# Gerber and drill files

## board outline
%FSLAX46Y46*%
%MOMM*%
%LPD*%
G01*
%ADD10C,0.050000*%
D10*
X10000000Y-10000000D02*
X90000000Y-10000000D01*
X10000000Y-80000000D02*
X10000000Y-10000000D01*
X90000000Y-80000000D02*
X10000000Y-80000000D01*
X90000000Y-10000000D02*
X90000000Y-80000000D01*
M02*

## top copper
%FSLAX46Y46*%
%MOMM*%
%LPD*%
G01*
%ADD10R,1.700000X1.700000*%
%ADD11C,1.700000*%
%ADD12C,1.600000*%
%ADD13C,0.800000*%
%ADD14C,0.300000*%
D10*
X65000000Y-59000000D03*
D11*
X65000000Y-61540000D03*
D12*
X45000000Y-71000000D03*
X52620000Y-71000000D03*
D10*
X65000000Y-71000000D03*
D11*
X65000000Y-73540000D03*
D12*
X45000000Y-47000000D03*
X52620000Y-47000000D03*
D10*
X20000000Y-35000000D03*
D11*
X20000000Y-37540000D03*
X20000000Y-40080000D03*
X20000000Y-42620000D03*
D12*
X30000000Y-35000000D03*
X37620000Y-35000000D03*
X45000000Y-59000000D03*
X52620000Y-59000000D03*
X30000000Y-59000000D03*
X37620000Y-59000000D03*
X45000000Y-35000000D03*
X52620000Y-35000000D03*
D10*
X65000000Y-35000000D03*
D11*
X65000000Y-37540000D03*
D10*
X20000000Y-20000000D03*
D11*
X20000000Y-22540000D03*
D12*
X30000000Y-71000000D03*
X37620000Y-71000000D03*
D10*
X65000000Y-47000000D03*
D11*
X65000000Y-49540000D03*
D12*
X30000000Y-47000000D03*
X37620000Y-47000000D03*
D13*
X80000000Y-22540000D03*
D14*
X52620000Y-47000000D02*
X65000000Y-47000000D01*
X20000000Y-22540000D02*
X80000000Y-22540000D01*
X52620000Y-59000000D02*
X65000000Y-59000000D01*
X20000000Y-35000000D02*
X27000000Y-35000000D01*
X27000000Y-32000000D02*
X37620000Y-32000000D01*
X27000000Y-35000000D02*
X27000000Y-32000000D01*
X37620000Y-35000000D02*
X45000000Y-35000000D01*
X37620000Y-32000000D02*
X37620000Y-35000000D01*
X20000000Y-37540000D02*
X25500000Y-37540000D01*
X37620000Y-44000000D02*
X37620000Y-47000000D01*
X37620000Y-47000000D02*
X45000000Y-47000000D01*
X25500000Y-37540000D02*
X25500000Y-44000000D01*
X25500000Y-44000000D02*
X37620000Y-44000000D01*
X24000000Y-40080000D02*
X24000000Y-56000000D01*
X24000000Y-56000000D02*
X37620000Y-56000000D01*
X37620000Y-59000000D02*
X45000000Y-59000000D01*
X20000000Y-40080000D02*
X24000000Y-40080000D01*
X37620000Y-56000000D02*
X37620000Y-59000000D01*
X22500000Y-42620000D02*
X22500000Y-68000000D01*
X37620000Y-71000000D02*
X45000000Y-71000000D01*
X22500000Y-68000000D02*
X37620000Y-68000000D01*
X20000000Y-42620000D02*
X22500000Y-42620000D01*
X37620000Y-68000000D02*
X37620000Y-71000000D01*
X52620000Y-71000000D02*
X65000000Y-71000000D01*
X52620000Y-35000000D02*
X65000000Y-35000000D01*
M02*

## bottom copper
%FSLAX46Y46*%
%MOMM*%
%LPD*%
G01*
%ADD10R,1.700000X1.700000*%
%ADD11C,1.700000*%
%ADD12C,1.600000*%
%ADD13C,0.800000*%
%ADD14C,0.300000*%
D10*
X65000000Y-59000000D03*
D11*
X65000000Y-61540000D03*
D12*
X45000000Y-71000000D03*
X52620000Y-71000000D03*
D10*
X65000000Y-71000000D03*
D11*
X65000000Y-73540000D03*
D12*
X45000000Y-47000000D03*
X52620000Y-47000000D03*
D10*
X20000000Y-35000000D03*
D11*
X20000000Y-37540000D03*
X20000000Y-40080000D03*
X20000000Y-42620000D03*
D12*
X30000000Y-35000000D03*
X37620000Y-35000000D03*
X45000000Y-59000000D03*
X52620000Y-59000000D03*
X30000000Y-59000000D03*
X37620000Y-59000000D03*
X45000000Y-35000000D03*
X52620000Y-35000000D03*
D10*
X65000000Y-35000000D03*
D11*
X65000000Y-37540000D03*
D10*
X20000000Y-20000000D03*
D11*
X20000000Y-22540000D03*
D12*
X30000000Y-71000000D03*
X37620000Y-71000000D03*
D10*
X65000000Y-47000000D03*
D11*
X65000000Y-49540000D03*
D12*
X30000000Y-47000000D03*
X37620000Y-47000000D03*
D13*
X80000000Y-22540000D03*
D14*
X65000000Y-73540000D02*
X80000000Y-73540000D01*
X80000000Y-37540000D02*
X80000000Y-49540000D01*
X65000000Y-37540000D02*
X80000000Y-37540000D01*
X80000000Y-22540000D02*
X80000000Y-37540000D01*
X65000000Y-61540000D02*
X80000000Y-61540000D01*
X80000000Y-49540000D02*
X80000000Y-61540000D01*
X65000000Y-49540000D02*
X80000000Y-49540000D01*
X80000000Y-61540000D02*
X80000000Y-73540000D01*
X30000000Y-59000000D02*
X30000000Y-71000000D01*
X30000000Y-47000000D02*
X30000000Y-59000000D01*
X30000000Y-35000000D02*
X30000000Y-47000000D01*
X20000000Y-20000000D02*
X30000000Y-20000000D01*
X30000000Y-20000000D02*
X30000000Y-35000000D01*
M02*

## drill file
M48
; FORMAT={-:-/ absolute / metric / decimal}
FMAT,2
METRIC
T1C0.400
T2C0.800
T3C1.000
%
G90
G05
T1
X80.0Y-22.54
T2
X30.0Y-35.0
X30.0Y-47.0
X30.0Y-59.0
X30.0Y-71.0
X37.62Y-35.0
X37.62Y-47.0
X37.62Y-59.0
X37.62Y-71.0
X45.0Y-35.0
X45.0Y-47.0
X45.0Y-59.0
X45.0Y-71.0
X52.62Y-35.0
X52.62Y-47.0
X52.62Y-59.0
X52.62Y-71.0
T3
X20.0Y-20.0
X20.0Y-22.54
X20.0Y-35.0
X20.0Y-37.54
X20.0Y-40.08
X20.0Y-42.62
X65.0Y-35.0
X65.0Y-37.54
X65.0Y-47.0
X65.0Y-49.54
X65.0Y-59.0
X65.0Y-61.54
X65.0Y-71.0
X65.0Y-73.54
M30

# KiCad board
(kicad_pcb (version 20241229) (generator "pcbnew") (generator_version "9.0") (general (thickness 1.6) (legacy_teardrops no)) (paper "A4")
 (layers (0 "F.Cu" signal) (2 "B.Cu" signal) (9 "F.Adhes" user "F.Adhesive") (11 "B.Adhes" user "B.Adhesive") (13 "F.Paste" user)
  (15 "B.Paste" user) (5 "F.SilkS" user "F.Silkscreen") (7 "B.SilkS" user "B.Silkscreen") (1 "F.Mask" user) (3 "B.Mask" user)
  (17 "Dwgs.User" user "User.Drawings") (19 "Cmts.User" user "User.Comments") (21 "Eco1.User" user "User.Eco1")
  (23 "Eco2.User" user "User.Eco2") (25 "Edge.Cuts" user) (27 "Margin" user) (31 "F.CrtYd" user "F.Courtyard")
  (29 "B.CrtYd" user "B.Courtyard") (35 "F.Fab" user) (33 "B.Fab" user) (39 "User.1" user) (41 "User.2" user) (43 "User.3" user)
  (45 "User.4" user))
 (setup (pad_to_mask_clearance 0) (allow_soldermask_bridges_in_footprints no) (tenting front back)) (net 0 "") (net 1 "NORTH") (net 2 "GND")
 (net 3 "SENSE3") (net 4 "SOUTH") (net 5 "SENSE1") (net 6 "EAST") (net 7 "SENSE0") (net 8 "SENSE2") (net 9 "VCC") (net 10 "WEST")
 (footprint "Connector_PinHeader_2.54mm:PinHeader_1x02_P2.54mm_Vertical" (layer "F.Cu") (at 65 59)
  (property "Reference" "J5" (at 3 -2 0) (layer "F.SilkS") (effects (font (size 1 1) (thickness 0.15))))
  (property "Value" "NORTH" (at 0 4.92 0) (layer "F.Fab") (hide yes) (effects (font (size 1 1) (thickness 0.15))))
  (pad "1" thru_hole rect (at 0 0) (size 1.7 1.7) (drill 1) (layers "*.Cu" "*.Mask") (remove_unused_layers no) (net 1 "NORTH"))
  (pad "2" thru_hole circle (at 0 2.54) (size 1.7 1.7) (drill 1) (layers "*.Cu" "*.Mask") (remove_unused_layers no) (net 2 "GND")))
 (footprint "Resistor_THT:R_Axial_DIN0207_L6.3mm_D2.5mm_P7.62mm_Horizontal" (layer "F.Cu") (at 45 71)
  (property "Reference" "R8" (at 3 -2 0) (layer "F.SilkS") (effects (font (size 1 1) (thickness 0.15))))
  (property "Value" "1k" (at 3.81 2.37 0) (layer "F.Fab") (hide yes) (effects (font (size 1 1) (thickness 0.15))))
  (pad "1" thru_hole circle (at 0 0) (size 1.6 1.6) (drill 0.8) (layers "*.Cu" "*.Mask") (remove_unused_layers no) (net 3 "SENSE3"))
  (pad "2" thru_hole circle (at 7.62 0) (size 1.6 1.6) (drill 0.8) (layers "*.Cu" "*.Mask") (remove_unused_layers no) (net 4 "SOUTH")))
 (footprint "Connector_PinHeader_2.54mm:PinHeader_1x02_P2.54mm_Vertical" (layer "F.Cu") (at 65 71)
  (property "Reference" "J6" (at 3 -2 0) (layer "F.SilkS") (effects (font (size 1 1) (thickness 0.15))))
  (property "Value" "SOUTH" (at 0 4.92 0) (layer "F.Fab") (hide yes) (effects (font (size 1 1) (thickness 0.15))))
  (pad "1" thru_hole rect (at 0 0) (size 1.7 1.7) (drill 1) (layers "*.Cu" "*.Mask") (remove_unused_layers no) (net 4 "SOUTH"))
  (pad "2" thru_hole circle (at 0 2.54) (size 1.7 1.7) (drill 1) (layers "*.Cu" "*.Mask") (remove_unused_layers no) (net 2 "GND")))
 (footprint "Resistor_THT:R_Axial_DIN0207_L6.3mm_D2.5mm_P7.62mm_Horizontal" (layer "F.Cu") (at 45 47)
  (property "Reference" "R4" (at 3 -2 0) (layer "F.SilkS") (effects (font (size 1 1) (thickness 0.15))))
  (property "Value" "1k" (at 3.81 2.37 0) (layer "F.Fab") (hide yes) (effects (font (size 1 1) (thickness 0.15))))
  (pad "1" thru_hole circle (at 0 0) (size 1.6 1.6) (drill 0.8) (layers "*.Cu" "*.Mask") (remove_unused_layers no) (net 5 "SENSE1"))
  (pad "2" thru_hole circle (at 7.62 0) (size 1.6 1.6) (drill 0.8) (layers "*.Cu" "*.Mask") (remove_unused_layers no) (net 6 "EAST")))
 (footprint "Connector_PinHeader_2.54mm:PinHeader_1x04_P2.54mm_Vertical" (layer "F.Cu") (at 20 35)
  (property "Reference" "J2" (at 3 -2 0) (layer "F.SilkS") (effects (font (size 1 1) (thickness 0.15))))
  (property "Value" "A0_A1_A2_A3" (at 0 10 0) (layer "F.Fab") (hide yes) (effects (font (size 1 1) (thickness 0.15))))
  (pad "1" thru_hole rect (at 0 0) (size 1.7 1.7) (drill 1) (layers "*.Cu" "*.Mask") (remove_unused_layers no) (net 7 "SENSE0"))
  (pad "2" thru_hole circle (at 0 2.54) (size 1.7 1.7) (drill 1) (layers "*.Cu" "*.Mask") (remove_unused_layers no) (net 5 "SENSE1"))
  (pad "3" thru_hole circle (at 0 5.08) (size 1.7 1.7) (drill 1) (layers "*.Cu" "*.Mask") (remove_unused_layers no) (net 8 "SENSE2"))
  (pad "4" thru_hole circle (at 0 7.62) (size 1.7 1.7) (drill 1) (layers "*.Cu" "*.Mask") (remove_unused_layers no) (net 3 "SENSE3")))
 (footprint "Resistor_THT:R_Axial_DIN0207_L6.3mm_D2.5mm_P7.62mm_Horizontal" (layer "F.Cu") (at 30 35)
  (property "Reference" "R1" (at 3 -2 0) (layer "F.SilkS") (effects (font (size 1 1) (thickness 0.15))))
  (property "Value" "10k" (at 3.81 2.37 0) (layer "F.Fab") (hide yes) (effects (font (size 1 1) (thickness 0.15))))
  (pad "1" thru_hole circle (at 0 0) (size 1.6 1.6) (drill 0.8) (layers "*.Cu" "*.Mask") (remove_unused_layers no) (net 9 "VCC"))
  (pad "2" thru_hole circle (at 7.62 0) (size 1.6 1.6) (drill 0.8) (layers "*.Cu" "*.Mask") (remove_unused_layers no) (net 7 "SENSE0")))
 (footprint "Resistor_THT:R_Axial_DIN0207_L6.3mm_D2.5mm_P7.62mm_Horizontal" (layer "F.Cu") (at 45 59)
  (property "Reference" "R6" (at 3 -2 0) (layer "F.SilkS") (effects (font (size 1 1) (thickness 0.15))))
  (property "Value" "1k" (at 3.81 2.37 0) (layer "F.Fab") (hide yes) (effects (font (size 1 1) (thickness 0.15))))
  (pad "1" thru_hole circle (at 0 0) (size 1.6 1.6) (drill 0.8) (layers "*.Cu" "*.Mask") (remove_unused_layers no) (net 8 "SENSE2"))
  (pad "2" thru_hole circle (at 7.62 0) (size 1.6 1.6) (drill 0.8) (layers "*.Cu" "*.Mask") (remove_unused_layers no) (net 1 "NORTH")))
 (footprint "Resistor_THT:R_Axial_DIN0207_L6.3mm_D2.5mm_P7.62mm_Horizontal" (layer "F.Cu") (at 30 59)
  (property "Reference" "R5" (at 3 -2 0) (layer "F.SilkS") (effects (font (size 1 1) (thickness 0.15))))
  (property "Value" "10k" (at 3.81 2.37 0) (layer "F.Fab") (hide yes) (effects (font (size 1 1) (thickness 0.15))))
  (pad "1" thru_hole circle (at 0 0) (size 1.6 1.6) (drill 0.8) (layers "*.Cu" "*.Mask") (remove_unused_layers no) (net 9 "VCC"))
  (pad "2" thru_hole circle (at 7.62 0) (size 1.6 1.6) (drill 0.8) (layers "*.Cu" "*.Mask") (remove_unused_layers no) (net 8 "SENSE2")))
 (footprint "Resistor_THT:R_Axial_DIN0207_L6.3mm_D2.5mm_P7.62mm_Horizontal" (layer "F.Cu") (at 45 35)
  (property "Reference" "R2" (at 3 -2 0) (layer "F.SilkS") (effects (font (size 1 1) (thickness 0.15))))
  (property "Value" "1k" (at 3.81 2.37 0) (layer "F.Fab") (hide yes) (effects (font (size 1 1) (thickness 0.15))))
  (pad "1" thru_hole circle (at 0 0) (size 1.6 1.6) (drill 0.8) (layers "*.Cu" "*.Mask") (remove_unused_layers no) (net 7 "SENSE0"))
  (pad "2" thru_hole circle (at 7.62 0) (size 1.6 1.6) (drill 0.8) (layers "*.Cu" "*.Mask") (remove_unused_layers no) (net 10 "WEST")))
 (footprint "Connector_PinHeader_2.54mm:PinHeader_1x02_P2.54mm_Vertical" (layer "F.Cu") (at 65 35)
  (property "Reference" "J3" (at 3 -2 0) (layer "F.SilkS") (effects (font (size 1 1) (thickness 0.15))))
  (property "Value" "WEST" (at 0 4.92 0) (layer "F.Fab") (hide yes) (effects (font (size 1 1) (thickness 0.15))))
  (pad "1" thru_hole rect (at 0 0) (size 1.7 1.7) (drill 1) (layers "*.Cu" "*.Mask") (remove_unused_layers no) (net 10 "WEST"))
  (pad "2" thru_hole circle (at 0 2.54) (size 1.7 1.7) (drill 1) (layers "*.Cu" "*.Mask") (remove_unused_layers no) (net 2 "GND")))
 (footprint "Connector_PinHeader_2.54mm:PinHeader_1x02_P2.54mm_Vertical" (layer "F.Cu") (at 20 20)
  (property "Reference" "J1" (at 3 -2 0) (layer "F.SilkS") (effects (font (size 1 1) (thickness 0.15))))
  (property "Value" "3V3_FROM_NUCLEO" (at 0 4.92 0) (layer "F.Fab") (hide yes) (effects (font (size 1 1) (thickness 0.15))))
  (pad "1" thru_hole rect (at 0 0) (size 1.7 1.7) (drill 1) (layers "*.Cu" "*.Mask") (remove_unused_layers no) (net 9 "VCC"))
  (pad "2" thru_hole circle (at 0 2.54) (size 1.7 1.7) (drill 1) (layers "*.Cu" "*.Mask") (remove_unused_layers no) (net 2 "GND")))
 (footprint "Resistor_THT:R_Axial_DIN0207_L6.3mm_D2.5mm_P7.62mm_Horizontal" (layer "F.Cu") (at 30 71)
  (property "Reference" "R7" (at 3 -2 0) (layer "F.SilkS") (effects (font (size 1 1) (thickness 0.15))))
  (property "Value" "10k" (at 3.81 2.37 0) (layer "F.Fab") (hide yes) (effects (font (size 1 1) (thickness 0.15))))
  (pad "1" thru_hole circle (at 0 0) (size 1.6 1.6) (drill 0.8) (layers "*.Cu" "*.Mask") (remove_unused_layers no) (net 9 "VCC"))
  (pad "2" thru_hole circle (at 7.62 0) (size 1.6 1.6) (drill 0.8) (layers "*.Cu" "*.Mask") (remove_unused_layers no) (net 3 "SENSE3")))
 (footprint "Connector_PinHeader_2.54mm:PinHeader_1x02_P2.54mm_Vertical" (layer "F.Cu") (at 65 47)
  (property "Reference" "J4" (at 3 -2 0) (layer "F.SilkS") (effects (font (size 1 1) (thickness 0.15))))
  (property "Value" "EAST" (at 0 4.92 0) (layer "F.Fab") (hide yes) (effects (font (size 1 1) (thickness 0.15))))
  (pad "1" thru_hole rect (at 0 0) (size 1.7 1.7) (drill 1) (layers "*.Cu" "*.Mask") (remove_unused_layers no) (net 6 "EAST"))
  (pad "2" thru_hole circle (at 0 2.54) (size 1.7 1.7) (drill 1) (layers "*.Cu" "*.Mask") (remove_unused_layers no) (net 2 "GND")))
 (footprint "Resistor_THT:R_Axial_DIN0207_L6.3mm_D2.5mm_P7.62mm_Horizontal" (layer "F.Cu") (at 30 47)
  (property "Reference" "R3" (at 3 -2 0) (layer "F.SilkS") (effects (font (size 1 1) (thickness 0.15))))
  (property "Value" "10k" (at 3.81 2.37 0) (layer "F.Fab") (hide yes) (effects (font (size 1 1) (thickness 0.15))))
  (pad "1" thru_hole circle (at 0 0) (size 1.6 1.6) (drill 0.8) (layers "*.Cu" "*.Mask") (remove_unused_layers no) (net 9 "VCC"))
  (pad "2" thru_hole circle (at 7.62 0) (size 1.6 1.6) (drill 0.8) (layers "*.Cu" "*.Mask") (remove_unused_layers no) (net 5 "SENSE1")))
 (gr_line (start 10 10) (end 90 10) (stroke (width 0.05) (type default)) (layer "Edge.Cuts"))
 (gr_line (start 10 80) (end 10 10) (stroke (width 0.05) (type default)) (layer "Edge.Cuts"))
 (gr_line (start 90 80) (end 10 80) (stroke (width 0.05) (type default)) (layer "Edge.Cuts"))
 (gr_line (start 90 10) (end 90 80) (stroke (width 0.05) (type default)) (layer "Edge.Cuts"))
 (segment (start 52.62 47) (end 65 47) (width 0.3) (layer "F.Cu") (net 6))
 (segment (start 20 22.54) (end 80 22.54) (width 0.3) (layer "F.Cu") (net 2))
 (via (at 80 22.54) (size 0.8) (drill 0.4) (layers "F.Cu" "B.Cu") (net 2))
 (segment (start 65 73.54) (end 80 73.54) (width 0.3) (layer "B.Cu") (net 2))
 (segment (start 80 37.54) (end 80 49.54) (width 0.3) (layer "B.Cu") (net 2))
 (segment (start 65 37.54) (end 80 37.54) (width 0.3) (layer "B.Cu") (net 2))
 (segment (start 80 22.54) (end 80 37.54) (width 0.3) (layer "B.Cu") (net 2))
 (segment (start 65 61.54) (end 80 61.54) (width 0.3) (layer "B.Cu") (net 2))
 (segment (start 80 49.54) (end 80 61.54) (width 0.3) (layer "B.Cu") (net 2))
 (segment (start 65 49.54) (end 80 49.54) (width 0.3) (layer "B.Cu") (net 2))
 (segment (start 80 61.54) (end 80 73.54) (width 0.3) (layer "B.Cu") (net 2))
 (segment (start 52.62 59) (end 65 59) (width 0.3) (layer "F.Cu") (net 1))
 (segment (start 20 35) (end 27 35) (width 0.3) (layer "F.Cu") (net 7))
 (segment (start 27 32) (end 37.62 32) (width 0.3) (layer "F.Cu") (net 7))
 (segment (start 27 35) (end 27 32) (width 0.3) (layer "F.Cu") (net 7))
 (segment (start 37.62 35) (end 45 35) (width 0.3) (layer "F.Cu") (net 7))
 (segment (start 37.62 32) (end 37.62 35) (width 0.3) (layer "F.Cu") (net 7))
 (segment (start 20 37.54) (end 25.5 37.54) (width 0.3) (layer "F.Cu") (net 5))
 (segment (start 37.62 44) (end 37.62 47) (width 0.3) (layer "F.Cu") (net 5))
 (segment (start 37.62 47) (end 45 47) (width 0.3) (layer "F.Cu") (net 5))
 (segment (start 25.5 37.54) (end 25.5 44) (width 0.3) (layer "F.Cu") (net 5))
 (segment (start 25.5 44) (end 37.62 44) (width 0.3) (layer "F.Cu") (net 5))
 (segment (start 24 40.08) (end 24 56) (width 0.3) (layer "F.Cu") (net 8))
 (segment (start 24 56) (end 37.62 56) (width 0.3) (layer "F.Cu") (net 8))
 (segment (start 37.62 59) (end 45 59) (width 0.3) (layer "F.Cu") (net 8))
 (segment (start 20 40.08) (end 24 40.08) (width 0.3) (layer "F.Cu") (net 8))
 (segment (start 37.62 56) (end 37.62 59) (width 0.3) (layer "F.Cu") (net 8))
 (segment (start 22.5 42.62) (end 22.5 68) (width 0.3) (layer "F.Cu") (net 3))
 (segment (start 37.62 71) (end 45 71) (width 0.3) (layer "F.Cu") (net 3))
 (segment (start 22.5 68) (end 37.62 68) (width 0.3) (layer "F.Cu") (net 3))
 (segment (start 20 42.62) (end 22.5 42.62) (width 0.3) (layer "F.Cu") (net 3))
 (segment (start 37.62 68) (end 37.62 71) (width 0.3) (layer "F.Cu") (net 3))
 (segment (start 52.62 71) (end 65 71) (width 0.3) (layer "F.Cu") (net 4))
 (segment (start 30 59) (end 30 71) (width 0.3) (layer "B.Cu") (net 9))
 (segment (start 30 47) (end 30 59) (width 0.3) (layer "B.Cu") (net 9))
 (segment (start 30 35) (end 30 47) (width 0.3) (layer "B.Cu") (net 9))
 (segment (start 20 20) (end 30 20) (width 0.3) (layer "B.Cu") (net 9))
 (segment (start 30 20) (end 30 35) (width 0.3) (layer "B.Cu") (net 9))
 (segment (start 52.62 35) (end 65 35) (width 0.3) (layer "F.Cu") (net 10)))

